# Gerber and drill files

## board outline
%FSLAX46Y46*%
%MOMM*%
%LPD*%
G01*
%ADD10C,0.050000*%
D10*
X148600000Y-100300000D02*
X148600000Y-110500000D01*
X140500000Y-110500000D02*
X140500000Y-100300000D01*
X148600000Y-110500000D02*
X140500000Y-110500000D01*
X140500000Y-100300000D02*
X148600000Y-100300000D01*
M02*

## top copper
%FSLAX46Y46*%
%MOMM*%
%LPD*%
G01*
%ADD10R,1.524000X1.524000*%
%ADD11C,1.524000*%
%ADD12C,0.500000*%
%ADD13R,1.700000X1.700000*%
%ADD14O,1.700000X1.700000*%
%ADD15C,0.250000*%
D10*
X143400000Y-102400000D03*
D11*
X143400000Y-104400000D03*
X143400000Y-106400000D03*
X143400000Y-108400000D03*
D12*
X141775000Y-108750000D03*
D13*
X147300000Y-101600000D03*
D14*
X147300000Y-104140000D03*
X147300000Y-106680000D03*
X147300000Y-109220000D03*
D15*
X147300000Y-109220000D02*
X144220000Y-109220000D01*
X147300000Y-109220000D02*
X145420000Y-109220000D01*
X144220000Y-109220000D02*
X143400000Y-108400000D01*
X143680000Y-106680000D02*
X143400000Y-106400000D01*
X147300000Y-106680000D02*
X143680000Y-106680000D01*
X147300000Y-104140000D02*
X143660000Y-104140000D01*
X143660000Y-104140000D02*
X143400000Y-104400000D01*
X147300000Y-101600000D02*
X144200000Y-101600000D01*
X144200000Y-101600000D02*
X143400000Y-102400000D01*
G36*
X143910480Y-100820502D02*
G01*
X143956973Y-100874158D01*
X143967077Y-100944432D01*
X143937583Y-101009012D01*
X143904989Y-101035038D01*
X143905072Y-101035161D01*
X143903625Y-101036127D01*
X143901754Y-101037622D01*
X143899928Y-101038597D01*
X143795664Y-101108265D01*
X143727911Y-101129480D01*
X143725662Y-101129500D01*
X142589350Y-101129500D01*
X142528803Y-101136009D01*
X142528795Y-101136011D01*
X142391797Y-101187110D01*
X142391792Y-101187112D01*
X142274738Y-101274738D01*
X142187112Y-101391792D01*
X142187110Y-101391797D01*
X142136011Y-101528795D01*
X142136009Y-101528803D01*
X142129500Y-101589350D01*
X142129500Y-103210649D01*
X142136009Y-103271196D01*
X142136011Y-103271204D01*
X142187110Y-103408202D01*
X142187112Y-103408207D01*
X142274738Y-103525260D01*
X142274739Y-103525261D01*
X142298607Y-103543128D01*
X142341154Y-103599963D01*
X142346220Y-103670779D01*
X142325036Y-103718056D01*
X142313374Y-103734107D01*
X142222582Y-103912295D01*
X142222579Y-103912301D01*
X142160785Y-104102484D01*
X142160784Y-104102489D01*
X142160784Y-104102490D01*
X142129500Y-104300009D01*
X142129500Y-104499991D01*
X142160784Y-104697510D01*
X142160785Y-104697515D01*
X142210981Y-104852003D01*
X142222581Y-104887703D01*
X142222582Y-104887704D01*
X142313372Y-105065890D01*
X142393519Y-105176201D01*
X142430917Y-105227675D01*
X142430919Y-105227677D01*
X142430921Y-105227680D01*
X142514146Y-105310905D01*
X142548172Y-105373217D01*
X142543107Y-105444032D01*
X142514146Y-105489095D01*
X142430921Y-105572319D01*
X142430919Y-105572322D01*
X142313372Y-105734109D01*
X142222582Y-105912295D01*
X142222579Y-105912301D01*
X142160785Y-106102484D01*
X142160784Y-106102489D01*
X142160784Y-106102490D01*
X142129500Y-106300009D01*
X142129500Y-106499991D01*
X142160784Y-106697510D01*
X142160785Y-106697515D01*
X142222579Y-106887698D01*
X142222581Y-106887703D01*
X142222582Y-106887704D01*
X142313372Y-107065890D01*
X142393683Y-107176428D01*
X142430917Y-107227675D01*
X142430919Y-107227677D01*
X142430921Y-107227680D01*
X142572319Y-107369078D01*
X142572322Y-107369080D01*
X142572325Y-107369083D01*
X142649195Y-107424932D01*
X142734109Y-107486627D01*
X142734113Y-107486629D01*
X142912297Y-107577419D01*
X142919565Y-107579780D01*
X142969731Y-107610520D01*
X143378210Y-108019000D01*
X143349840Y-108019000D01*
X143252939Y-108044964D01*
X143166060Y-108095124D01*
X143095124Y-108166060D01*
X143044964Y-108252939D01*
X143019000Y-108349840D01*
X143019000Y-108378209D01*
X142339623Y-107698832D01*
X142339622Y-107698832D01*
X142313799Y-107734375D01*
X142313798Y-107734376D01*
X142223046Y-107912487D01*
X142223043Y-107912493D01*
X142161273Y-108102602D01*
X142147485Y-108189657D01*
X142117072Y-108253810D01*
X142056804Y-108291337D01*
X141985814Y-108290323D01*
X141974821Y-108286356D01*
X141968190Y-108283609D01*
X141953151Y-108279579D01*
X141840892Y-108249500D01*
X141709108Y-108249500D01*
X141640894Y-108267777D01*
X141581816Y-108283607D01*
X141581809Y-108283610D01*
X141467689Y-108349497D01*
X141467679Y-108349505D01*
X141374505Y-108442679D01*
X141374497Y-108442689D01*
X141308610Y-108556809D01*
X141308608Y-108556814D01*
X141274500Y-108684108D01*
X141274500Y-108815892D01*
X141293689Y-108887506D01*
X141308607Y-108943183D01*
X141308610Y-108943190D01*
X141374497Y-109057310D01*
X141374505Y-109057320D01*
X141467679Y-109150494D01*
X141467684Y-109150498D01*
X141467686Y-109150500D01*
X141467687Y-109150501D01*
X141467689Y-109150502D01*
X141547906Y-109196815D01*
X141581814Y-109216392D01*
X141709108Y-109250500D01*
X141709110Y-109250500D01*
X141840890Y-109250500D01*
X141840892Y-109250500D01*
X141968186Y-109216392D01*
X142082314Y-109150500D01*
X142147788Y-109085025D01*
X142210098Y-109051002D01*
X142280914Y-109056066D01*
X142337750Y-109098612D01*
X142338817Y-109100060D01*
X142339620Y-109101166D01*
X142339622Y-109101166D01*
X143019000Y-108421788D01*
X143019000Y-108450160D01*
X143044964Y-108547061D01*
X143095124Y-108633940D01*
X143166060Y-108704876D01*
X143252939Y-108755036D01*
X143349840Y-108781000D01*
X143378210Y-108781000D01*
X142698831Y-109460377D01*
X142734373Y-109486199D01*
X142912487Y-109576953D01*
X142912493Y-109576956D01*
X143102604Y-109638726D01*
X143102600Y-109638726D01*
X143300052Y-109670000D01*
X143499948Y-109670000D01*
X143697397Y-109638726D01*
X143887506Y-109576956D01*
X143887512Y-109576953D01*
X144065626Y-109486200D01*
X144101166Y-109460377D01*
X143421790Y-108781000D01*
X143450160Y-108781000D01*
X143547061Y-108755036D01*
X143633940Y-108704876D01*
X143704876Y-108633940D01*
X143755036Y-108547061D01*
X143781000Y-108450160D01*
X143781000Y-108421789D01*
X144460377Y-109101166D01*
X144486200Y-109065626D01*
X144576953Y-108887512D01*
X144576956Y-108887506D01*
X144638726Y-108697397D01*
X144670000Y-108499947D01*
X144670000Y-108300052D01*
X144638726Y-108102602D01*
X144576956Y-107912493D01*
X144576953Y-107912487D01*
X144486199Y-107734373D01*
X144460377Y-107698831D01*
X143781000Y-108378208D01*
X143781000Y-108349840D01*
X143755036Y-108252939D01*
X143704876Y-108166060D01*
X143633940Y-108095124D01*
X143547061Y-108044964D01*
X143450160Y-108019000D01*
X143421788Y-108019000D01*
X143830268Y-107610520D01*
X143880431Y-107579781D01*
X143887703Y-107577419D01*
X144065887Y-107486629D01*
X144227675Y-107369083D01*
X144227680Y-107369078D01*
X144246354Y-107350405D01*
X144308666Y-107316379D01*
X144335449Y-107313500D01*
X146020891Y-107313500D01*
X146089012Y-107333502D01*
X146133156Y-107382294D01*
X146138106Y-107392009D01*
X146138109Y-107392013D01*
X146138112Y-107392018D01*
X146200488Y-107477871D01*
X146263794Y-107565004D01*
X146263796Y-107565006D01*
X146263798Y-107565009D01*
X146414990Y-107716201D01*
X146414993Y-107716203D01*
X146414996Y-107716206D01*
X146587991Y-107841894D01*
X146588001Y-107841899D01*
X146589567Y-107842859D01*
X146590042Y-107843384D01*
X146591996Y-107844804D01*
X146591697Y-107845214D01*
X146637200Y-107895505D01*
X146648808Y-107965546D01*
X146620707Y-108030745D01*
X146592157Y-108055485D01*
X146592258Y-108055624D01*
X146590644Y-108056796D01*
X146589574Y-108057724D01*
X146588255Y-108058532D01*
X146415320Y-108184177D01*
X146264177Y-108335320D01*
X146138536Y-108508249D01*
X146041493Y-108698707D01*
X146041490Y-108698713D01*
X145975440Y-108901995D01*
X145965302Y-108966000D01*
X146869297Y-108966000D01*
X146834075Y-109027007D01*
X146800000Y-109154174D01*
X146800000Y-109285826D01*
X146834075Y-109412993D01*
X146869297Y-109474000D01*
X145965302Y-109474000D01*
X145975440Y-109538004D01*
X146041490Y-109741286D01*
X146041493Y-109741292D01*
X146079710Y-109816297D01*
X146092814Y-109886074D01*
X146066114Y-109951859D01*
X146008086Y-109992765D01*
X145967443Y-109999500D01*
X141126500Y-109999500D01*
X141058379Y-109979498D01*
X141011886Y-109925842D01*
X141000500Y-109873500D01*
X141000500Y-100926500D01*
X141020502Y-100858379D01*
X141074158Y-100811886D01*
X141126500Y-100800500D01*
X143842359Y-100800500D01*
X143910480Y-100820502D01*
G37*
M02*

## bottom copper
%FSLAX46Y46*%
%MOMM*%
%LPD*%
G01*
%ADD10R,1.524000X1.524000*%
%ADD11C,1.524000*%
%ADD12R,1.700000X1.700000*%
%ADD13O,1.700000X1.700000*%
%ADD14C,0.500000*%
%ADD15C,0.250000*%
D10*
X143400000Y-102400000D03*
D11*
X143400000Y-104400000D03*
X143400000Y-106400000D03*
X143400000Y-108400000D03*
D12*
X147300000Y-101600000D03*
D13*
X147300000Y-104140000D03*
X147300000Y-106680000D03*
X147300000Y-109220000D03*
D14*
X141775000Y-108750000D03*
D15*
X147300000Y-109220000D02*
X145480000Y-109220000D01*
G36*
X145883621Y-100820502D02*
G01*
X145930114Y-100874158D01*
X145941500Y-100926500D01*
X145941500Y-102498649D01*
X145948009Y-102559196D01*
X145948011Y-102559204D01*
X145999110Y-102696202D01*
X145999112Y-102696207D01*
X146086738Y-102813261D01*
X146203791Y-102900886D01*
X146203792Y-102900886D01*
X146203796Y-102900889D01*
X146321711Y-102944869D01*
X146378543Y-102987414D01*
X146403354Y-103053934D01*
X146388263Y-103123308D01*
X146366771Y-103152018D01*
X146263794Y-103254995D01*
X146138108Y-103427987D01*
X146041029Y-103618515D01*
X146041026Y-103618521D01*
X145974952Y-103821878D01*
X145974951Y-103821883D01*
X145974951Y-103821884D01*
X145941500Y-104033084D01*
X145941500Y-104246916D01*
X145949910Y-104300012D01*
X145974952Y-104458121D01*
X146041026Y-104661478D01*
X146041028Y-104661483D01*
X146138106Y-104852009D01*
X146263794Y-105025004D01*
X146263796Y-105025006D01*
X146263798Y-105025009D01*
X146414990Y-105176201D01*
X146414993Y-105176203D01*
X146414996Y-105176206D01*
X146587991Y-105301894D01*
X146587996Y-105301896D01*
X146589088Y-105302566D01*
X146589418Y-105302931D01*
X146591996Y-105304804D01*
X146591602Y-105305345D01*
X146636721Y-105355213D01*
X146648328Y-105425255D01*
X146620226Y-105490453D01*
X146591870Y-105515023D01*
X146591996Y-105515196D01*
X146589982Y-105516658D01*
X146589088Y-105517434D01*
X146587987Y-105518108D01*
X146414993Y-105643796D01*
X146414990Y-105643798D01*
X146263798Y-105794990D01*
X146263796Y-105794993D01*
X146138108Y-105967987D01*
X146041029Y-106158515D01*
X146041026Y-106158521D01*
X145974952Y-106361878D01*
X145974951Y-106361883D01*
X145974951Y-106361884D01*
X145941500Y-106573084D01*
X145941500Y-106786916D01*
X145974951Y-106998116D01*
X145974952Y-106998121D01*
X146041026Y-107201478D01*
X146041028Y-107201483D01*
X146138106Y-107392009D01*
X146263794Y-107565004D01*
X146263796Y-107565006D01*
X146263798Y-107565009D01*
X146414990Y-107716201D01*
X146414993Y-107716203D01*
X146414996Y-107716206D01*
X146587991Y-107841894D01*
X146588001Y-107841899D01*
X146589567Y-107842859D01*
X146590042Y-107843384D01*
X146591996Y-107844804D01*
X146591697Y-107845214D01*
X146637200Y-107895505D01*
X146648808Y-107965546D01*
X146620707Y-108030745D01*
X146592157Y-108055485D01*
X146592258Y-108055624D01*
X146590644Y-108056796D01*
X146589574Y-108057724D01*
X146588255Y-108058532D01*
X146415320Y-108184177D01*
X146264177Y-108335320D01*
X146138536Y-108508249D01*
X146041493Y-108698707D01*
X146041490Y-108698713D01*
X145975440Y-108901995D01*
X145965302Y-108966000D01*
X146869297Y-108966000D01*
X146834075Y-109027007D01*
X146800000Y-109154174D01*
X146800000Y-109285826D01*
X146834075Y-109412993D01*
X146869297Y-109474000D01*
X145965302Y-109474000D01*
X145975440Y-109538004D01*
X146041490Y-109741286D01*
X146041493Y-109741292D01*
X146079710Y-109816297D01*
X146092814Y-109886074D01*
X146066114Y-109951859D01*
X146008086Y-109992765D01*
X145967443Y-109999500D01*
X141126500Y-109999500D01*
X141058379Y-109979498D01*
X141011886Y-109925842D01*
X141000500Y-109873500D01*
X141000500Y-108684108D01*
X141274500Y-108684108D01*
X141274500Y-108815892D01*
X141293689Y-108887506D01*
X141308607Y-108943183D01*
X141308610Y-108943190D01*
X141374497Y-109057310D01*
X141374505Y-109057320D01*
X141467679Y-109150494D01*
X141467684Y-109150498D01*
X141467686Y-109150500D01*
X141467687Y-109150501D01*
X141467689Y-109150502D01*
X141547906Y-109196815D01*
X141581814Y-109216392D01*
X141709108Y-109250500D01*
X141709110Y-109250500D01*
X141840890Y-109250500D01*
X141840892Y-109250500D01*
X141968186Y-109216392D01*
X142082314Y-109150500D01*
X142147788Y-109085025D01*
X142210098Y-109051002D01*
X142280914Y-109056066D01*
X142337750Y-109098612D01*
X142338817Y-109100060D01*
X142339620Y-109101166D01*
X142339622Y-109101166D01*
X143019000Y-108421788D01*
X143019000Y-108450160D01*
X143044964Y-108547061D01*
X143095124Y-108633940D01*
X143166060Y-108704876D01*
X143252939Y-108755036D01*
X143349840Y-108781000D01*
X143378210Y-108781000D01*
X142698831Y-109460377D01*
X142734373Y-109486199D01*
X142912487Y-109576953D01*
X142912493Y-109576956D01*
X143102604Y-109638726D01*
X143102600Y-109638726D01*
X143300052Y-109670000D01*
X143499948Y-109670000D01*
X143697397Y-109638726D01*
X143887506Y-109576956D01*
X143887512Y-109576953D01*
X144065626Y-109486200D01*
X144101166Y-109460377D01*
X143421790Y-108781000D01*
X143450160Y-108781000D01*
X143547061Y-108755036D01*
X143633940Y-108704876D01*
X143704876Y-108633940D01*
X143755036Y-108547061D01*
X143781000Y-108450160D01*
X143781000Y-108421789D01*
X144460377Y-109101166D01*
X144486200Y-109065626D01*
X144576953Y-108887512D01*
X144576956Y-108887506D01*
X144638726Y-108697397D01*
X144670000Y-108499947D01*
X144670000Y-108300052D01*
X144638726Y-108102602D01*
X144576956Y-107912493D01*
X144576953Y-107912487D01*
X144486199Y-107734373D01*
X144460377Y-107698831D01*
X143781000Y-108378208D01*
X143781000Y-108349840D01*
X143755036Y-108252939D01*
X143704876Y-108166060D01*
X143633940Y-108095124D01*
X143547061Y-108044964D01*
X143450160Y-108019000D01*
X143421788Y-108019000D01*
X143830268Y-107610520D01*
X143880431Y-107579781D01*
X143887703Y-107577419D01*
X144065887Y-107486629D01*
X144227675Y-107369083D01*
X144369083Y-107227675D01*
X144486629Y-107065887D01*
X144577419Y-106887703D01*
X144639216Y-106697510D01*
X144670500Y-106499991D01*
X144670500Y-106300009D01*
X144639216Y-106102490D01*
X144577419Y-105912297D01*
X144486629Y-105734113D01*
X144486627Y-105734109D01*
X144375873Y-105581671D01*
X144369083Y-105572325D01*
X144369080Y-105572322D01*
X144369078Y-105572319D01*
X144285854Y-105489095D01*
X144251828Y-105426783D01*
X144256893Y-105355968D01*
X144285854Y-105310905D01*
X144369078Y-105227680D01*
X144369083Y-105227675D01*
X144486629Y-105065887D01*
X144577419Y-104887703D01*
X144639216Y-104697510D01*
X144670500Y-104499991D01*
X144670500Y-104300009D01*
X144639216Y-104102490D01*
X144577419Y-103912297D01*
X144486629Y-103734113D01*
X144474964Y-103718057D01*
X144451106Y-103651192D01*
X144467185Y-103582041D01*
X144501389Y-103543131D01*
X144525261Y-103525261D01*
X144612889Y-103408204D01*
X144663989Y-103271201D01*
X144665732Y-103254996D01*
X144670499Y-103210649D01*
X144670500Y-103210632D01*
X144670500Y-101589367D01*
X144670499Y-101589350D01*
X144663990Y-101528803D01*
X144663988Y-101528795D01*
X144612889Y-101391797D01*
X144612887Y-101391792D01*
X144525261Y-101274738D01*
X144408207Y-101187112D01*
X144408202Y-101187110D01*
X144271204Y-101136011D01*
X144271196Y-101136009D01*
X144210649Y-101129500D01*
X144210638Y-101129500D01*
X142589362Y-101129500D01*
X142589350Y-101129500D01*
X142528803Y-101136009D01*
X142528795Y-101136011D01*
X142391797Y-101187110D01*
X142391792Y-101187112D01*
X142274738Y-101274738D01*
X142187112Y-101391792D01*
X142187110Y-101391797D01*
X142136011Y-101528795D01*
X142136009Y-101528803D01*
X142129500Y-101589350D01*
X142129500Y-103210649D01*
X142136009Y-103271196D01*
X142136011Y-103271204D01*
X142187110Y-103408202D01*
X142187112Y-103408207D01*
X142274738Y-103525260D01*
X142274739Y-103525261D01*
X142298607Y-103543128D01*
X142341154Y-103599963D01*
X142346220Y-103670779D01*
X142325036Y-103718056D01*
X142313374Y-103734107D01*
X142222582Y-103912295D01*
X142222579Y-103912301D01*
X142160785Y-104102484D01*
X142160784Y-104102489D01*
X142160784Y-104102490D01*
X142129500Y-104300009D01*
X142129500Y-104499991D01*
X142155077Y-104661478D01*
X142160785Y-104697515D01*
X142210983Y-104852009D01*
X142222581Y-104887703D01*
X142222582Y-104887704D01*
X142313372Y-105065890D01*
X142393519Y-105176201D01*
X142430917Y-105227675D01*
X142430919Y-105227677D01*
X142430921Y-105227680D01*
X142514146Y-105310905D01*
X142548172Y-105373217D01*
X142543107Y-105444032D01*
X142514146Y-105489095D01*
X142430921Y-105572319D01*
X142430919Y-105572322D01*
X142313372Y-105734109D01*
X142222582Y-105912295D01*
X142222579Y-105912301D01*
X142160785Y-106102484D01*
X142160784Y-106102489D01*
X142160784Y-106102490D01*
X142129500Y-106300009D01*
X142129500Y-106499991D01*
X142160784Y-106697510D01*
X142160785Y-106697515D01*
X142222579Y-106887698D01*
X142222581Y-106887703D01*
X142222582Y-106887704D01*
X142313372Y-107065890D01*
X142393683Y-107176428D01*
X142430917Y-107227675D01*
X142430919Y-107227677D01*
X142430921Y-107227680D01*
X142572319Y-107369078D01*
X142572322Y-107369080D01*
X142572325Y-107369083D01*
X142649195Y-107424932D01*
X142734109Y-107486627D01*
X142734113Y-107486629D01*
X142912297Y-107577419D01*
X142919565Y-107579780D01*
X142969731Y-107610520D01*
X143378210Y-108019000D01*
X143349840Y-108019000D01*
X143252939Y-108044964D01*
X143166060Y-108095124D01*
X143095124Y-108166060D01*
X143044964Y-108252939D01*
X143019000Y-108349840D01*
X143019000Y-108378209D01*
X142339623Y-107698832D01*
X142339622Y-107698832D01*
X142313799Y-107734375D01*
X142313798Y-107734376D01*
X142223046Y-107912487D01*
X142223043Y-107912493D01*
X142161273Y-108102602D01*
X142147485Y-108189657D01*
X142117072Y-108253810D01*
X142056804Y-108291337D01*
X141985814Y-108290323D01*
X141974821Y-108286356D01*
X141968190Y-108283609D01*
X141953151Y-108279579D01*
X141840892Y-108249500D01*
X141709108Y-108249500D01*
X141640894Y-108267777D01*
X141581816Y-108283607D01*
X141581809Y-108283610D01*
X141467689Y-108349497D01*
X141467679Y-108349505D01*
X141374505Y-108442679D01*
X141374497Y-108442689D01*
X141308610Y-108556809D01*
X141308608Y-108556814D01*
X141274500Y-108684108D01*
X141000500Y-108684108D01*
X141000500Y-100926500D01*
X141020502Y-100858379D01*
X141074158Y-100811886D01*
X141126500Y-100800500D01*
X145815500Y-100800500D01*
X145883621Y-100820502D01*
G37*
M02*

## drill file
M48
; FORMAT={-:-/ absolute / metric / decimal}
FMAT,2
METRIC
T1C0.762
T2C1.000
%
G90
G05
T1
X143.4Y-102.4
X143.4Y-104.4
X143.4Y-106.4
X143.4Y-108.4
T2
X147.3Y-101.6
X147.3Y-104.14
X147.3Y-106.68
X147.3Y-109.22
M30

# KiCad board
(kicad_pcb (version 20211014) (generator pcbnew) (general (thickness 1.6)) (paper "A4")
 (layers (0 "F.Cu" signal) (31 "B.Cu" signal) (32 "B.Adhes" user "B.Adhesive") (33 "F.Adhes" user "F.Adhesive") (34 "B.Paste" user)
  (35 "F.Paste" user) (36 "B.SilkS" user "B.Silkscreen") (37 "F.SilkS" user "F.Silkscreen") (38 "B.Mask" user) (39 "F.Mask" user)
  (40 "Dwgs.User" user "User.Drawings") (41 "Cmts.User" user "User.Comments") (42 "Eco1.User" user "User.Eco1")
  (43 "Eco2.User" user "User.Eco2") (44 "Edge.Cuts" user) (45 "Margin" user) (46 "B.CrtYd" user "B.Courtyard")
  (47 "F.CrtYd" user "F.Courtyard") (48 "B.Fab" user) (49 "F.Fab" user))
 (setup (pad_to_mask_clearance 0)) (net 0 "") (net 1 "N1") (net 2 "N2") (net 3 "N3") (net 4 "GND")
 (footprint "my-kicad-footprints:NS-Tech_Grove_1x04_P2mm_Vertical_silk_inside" (layer "F.Cu") (at 143.4 102.4)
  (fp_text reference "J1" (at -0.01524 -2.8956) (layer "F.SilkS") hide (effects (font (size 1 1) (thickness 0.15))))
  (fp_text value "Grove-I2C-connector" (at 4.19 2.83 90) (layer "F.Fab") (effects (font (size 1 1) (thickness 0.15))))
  (pad "1" thru_hole rect locked (at 0 0) (size 1.524 1.524) (drill 0.762) (layers *.Cu *.Mask) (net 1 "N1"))
  (pad "2" thru_hole circle locked (at 0 2) (size 1.524 1.524) (drill 0.762) (layers *.Cu *.Mask) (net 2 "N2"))
  (pad "3" thru_hole circle locked (at 0 4) (size 1.524 1.524) (drill 0.762) (layers *.Cu *.Mask) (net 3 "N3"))
  (pad "4" thru_hole circle locked (at 0 6) (size 1.524 1.524) (drill 0.762) (layers *.Cu *.Mask) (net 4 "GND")))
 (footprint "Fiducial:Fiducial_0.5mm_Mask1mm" (layer "F.Cu") (at 141.775 108.75)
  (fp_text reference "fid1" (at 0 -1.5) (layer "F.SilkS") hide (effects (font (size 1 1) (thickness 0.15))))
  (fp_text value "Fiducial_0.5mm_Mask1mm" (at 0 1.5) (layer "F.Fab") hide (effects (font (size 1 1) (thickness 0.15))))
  (pad "" smd circle locked (at 0 0) (size 0.5 0.5) (layers "F.Cu" "F.Mask") (solder_mask_margin 0.25) (clearance 0.25)))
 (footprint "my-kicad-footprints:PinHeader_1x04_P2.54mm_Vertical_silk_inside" (layer "B.Cu") (at 147.3 101.6 180)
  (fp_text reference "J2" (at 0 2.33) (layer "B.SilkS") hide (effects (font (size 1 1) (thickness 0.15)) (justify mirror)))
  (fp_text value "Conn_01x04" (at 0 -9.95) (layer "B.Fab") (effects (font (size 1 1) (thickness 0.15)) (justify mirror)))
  (pad "1" thru_hole rect locked (at 0 0 180) (size 1.7 1.7) (drill 1) (layers *.Cu *.Mask) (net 1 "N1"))
  (pad "2" thru_hole oval locked (at 0 -2.54 180) (size 1.7 1.7) (drill 1) (layers *.Cu *.Mask) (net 2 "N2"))
  (pad "3" thru_hole oval locked (at 0 -5.08 180) (size 1.7 1.7) (drill 1) (layers *.Cu *.Mask) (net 3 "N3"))
  (pad "4" thru_hole oval locked (at 0 -7.62 180) (size 1.7 1.7) (drill 1) (layers *.Cu *.Mask) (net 4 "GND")))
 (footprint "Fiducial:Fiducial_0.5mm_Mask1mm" (layer "B.Cu") (at 141.775 108.75)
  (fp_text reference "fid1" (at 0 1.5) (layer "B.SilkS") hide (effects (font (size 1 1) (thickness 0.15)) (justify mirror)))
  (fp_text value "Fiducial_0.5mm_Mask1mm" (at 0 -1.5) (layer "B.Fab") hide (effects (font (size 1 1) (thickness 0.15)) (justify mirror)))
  (pad "" smd circle locked (at 0 0) (size 0.5 0.5) (layers "B.Cu" "B.Mask") (solder_mask_margin 0.25) (clearance 0.25)))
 (gr_line (start 148.6 100.3) (end 148.6 110.5) (layer "Edge.Cuts") (width 0.05))
 (gr_line (start 140.5 110.5) (end 140.5 100.3) (layer "Edge.Cuts") (width 0.05))
 (gr_line (start 148.6 110.5) (end 140.5 110.5) (layer "Edge.Cuts") (width 0.05))
 (gr_line (start 140.5 100.3) (end 148.6 100.3) (layer "Edge.Cuts") (width 0.05))
 (segment (start 147.3 109.22) (end 144.22 109.22) (width 0.25) (layer "F.Cu") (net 4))
 (segment (start 147.3 109.22) (end 145.42 109.22) (width 0.25) (layer "F.Cu") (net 4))
 (segment (start 144.22 109.22) (end 143.4 108.4) (width 0.25) (layer "F.Cu") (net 4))
 (segment (start 147.3 109.22) (end 145.48 109.22) (width 0.25) (layer "B.Cu") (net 4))
 (segment (start 143.68 106.68) (end 143.4 106.4) (width 0.25) (layer "F.Cu") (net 3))
 (segment (start 147.3 106.68) (end 143.68 106.68) (width 0.25) (layer "F.Cu") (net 3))
 (segment (start 147.3 104.14) (end 143.66 104.14) (width 0.25) (layer "F.Cu") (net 2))
 (segment (start 143.66 104.14) (end 143.4 104.4) (width 0.25) (layer "F.Cu") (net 2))
 (segment (start 147.3 101.6) (end 144.2 101.6) (width 0.25) (layer "F.Cu") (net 1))
 (segment (start 144.2 101.6) (end 143.4 102.4) (width 0.25) (layer "F.Cu") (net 1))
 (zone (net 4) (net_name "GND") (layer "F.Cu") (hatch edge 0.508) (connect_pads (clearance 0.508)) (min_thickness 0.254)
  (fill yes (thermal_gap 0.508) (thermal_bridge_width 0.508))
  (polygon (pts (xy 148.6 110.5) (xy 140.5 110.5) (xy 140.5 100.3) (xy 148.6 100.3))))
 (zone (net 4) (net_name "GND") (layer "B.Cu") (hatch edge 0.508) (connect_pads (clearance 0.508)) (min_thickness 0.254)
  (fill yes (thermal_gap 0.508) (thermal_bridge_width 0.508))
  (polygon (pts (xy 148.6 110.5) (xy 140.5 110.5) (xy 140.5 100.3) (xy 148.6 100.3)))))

